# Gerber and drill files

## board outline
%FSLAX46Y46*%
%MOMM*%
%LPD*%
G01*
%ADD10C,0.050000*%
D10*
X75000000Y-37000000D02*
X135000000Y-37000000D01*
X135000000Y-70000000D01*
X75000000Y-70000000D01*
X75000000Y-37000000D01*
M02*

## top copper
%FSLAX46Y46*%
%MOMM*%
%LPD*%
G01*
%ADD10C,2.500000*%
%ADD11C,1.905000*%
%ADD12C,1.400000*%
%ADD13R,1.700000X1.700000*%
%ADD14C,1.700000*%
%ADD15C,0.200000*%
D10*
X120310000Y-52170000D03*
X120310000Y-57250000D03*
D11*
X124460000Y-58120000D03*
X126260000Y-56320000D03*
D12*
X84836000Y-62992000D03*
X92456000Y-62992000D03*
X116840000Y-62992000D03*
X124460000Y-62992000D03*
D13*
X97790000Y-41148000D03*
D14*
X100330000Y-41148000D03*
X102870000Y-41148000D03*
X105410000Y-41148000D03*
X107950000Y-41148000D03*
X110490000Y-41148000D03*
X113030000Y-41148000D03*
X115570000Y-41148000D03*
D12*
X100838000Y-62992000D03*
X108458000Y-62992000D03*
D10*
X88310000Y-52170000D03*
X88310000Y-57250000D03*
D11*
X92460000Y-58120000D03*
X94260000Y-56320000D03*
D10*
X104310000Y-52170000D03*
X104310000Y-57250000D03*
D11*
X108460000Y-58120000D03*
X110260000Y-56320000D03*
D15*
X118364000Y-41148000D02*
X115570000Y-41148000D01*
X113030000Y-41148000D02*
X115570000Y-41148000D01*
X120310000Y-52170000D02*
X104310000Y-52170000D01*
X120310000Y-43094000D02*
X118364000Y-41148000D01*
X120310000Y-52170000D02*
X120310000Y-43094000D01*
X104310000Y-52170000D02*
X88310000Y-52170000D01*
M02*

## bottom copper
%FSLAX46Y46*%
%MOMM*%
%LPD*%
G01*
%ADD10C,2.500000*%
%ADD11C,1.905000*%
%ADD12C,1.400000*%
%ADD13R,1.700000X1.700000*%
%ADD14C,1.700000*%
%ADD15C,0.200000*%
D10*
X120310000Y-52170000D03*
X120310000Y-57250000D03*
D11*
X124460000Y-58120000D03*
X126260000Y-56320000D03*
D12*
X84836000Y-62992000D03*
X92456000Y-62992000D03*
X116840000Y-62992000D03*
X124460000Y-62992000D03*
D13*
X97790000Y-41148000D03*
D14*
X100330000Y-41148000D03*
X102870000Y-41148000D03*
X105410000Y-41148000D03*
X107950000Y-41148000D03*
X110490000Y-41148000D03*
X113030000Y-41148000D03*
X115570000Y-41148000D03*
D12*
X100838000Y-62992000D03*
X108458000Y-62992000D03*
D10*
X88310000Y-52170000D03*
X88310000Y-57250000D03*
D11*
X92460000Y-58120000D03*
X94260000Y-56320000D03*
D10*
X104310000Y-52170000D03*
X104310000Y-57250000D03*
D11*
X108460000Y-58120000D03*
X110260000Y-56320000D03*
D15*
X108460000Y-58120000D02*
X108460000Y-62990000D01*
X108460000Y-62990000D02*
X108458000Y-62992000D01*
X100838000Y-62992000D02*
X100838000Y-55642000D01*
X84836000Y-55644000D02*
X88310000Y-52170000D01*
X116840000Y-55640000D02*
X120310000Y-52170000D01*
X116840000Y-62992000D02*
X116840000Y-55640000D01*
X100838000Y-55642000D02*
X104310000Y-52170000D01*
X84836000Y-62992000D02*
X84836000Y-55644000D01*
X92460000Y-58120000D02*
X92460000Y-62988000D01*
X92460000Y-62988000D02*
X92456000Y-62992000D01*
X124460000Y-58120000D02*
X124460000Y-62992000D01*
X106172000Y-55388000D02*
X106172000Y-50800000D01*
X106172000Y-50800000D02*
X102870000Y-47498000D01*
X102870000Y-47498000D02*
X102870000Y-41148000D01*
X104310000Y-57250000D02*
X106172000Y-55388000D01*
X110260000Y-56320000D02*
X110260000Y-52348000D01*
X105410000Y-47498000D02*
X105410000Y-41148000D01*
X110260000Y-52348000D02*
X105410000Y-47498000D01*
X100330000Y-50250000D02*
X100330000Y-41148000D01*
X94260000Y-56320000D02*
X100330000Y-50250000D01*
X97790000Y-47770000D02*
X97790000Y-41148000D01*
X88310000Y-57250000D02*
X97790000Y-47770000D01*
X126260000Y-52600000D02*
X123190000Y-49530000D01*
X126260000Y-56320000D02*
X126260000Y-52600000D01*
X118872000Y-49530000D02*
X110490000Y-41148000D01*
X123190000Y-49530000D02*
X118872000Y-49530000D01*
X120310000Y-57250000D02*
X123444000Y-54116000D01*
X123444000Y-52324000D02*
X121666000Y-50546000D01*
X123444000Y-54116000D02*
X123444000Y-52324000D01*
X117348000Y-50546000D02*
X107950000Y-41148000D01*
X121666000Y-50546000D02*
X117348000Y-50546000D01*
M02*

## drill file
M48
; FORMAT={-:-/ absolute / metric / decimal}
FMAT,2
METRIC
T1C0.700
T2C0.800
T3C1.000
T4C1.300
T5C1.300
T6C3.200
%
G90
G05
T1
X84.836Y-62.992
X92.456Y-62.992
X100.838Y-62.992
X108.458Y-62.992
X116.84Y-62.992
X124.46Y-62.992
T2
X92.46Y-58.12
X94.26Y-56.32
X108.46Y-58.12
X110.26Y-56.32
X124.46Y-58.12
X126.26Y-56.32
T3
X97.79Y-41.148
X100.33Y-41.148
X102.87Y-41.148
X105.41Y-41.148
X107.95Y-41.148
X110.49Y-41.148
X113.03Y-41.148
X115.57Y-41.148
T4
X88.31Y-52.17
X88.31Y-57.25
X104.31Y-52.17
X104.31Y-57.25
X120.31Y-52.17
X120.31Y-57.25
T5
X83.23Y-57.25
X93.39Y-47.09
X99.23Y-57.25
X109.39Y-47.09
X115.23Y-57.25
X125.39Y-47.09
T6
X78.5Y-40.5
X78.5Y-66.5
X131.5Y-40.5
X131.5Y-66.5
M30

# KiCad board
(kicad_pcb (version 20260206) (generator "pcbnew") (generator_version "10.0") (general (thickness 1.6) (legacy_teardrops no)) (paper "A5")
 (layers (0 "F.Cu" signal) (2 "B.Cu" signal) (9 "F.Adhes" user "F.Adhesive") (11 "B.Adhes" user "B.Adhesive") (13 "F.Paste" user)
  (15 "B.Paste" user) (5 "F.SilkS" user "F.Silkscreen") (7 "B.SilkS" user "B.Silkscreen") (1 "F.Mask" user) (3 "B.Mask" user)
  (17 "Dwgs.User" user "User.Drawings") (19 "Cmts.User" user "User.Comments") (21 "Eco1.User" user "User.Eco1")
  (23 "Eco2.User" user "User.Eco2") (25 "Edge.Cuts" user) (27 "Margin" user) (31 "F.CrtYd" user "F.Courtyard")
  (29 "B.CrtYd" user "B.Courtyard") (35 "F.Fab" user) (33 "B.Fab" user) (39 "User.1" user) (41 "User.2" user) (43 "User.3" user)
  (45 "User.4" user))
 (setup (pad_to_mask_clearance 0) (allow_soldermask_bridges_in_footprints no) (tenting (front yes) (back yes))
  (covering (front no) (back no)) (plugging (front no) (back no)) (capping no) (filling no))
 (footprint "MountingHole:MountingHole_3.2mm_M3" (layer "F.Cu") (at 78.5 40.5)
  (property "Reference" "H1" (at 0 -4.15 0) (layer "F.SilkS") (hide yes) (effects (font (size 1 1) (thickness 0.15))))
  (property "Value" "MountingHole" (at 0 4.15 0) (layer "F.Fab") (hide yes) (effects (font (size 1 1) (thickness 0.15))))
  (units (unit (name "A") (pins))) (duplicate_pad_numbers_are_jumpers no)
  (pad "" np_thru_hole circle (at 0 0) (size 3.2 3.2) (drill 3.2) (layers "*.Cu" "*.Mask")))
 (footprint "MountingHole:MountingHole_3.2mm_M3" (layer "F.Cu") (at 131.5 66.5)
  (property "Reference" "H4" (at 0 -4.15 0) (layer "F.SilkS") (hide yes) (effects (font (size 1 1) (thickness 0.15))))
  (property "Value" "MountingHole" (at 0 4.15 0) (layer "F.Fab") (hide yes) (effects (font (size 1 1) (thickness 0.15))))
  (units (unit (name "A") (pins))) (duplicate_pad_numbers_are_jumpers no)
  (pad "" np_thru_hole circle (at 0 0) (size 3.2 3.2) (drill 3.2) (layers "*.Cu" "*.Mask")))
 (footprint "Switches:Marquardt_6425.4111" (layer "F.Cu") (at 120.31 52.17 180)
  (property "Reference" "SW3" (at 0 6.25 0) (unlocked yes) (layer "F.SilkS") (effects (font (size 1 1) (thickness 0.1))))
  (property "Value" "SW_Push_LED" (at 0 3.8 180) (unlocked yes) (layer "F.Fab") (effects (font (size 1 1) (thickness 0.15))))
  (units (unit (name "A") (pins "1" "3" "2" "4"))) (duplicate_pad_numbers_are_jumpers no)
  (pad "" np_thru_hole circle (at -5.08 5.08 180) (size 1.3 1.3) (drill 1.3) (layers "*.Cu" "*.Mask"))
  (pad "" np_thru_hole circle (at 5.08 -5.08 180) (size 1.3 1.3) (drill 1.3) (layers "*.Cu" "*.Mask"))
  (pad "1" thru_hole circle (at 0 0 180) (size 2.5 2.5) (drill 1.3) (layers "*.Cu" "*.Mask") (remove_unused_layers no) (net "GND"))
  (pad "2" thru_hole circle (at 0 -5.08 180) (size 2.5 2.5) (drill 1.3) (layers "*.Cu" "*.Mask") (remove_unused_layers no)
   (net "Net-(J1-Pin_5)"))
  (pad "3" thru_hole circle (at -4.15 -5.95 180) (size 1.905 1.905) (drill 0.8) (layers "*.Cu" "*.Mask") (remove_unused_layers no)
   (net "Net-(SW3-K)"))
  (pad "4" thru_hole circle (at -5.95 -4.15 180) (size 1.905 1.905) (drill 0.8) (layers "*.Cu" "*.Mask") (remove_unused_layers no)
   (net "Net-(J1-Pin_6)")))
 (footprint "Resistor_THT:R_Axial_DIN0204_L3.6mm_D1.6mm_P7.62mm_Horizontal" (layer "F.Cu") (at 84.836 62.992)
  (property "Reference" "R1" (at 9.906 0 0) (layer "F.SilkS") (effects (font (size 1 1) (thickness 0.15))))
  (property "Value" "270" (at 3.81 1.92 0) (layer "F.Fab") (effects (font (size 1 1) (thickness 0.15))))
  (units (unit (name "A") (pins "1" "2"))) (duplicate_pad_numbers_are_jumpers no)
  (pad "1" thru_hole circle (at 0 0) (size 1.4 1.4) (drill 0.7) (layers "*.Cu" "*.Mask") (remove_unused_layers no) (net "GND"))
  (pad "2" thru_hole circle (at 7.62 0) (size 1.4 1.4) (drill 0.7) (layers "*.Cu" "*.Mask") (remove_unused_layers no) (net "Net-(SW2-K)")))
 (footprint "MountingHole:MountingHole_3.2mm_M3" (layer "F.Cu") (at 131.5 40.5)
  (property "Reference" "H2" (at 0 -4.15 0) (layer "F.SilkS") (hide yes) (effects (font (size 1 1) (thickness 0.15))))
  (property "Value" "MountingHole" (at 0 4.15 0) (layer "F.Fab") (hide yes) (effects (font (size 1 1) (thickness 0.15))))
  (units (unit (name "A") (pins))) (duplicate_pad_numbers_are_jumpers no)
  (pad "" np_thru_hole circle (at 0 0) (size 3.2 3.2) (drill 3.2) (layers "*.Cu" "*.Mask")))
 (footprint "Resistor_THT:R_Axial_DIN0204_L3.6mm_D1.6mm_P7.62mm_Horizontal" (layer "F.Cu") (at 116.84 62.992)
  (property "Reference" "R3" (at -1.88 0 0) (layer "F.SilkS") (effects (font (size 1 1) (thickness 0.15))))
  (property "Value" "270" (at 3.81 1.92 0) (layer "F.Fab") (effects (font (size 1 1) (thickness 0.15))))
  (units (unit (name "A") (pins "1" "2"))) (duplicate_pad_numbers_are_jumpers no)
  (pad "1" thru_hole circle (at 0 0) (size 1.4 1.4) (drill 0.7) (layers "*.Cu" "*.Mask") (remove_unused_layers no) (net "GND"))
  (pad "2" thru_hole circle (at 7.62 0) (size 1.4 1.4) (drill 0.7) (layers "*.Cu" "*.Mask") (remove_unused_layers no) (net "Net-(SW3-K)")))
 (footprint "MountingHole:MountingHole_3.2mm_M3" (layer "F.Cu") (at 78.5 66.5)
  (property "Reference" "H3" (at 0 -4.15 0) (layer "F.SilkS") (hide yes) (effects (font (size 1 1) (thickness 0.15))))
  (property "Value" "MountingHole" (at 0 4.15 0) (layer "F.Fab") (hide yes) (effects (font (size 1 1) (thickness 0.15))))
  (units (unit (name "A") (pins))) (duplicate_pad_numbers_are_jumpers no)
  (pad "" np_thru_hole circle (at 0 0) (size 3.2 3.2) (drill 3.2) (layers "*.Cu" "*.Mask")))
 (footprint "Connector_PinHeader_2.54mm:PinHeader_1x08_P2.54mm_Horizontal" (layer "F.Cu") (at 97.79 41.148 90)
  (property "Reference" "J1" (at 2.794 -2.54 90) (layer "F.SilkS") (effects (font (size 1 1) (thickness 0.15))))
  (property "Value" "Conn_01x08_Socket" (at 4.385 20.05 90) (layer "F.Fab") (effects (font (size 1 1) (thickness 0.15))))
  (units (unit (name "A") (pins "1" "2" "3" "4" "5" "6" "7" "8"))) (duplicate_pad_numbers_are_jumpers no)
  (pad "1" thru_hole rect (at 0 0 90) (size 1.7 1.7) (drill 1) (layers "*.Cu" "*.Mask") (remove_unused_layers no) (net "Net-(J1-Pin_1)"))
  (pad "2" thru_hole circle (at 0 2.54 90) (size 1.7 1.7) (drill 1) (layers "*.Cu" "*.Mask") (remove_unused_layers no)
   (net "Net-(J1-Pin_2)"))
  (pad "3" thru_hole circle (at 0 5.08 90) (size 1.7 1.7) (drill 1) (layers "*.Cu" "*.Mask") (remove_unused_layers no)
   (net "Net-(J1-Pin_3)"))
  (pad "4" thru_hole circle (at 0 7.62 90) (size 1.7 1.7) (drill 1) (layers "*.Cu" "*.Mask") (remove_unused_layers no)
   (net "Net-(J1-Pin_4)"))
  (pad "5" thru_hole circle (at 0 10.16 90) (size 1.7 1.7) (drill 1) (layers "*.Cu" "*.Mask") (remove_unused_layers no)
   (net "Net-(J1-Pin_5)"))
  (pad "6" thru_hole circle (at 0 12.7 90) (size 1.7 1.7) (drill 1) (layers "*.Cu" "*.Mask") (remove_unused_layers no)
   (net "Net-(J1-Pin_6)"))
  (pad "7" thru_hole circle (at 0 15.24 90) (size 1.7 1.7) (drill 1) (layers "*.Cu" "*.Mask") (remove_unused_layers no) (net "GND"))
  (pad "8" thru_hole circle (at 0 17.78 90) (size 1.7 1.7) (drill 1) (layers "*.Cu" "*.Mask") (remove_unused_layers no) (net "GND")))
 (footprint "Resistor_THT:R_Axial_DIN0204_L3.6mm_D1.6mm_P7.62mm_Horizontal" (layer "F.Cu") (at 100.838 62.992)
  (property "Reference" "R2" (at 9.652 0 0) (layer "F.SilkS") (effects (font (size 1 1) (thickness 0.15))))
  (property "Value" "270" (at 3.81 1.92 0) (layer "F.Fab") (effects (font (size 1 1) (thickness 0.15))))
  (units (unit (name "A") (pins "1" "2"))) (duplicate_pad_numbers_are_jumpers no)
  (pad "1" thru_hole circle (at 0 0) (size 1.4 1.4) (drill 0.7) (layers "*.Cu" "*.Mask") (remove_unused_layers no) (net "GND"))
  (pad "2" thru_hole circle (at 7.62 0) (size 1.4 1.4) (drill 0.7) (layers "*.Cu" "*.Mask") (remove_unused_layers no) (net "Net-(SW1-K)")))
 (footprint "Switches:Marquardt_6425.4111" (layer "F.Cu") (at 88.31 52.17 180)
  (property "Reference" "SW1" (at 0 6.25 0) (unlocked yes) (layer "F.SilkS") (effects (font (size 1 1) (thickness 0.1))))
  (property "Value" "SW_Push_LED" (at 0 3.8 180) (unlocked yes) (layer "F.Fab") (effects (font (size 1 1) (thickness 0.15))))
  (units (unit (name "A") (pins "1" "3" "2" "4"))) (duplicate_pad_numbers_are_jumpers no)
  (pad "" np_thru_hole circle (at -5.08 5.08 180) (size 1.3 1.3) (drill 1.3) (layers "*.Cu" "*.Mask"))
  (pad "" np_thru_hole circle (at 5.08 -5.08 180) (size 1.3 1.3) (drill 1.3) (layers "*.Cu" "*.Mask"))
  (pad "1" thru_hole circle (at 0 0 180) (size 2.5 2.5) (drill 1.3) (layers "*.Cu" "*.Mask") (remove_unused_layers no) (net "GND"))
  (pad "2" thru_hole circle (at 0 -5.08 180) (size 2.5 2.5) (drill 1.3) (layers "*.Cu" "*.Mask") (remove_unused_layers no)
   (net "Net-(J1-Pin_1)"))
  (pad "3" thru_hole circle (at -4.15 -5.95 180) (size 1.905 1.905) (drill 0.8) (layers "*.Cu" "*.Mask") (remove_unused_layers no)
   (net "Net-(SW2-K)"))
  (pad "4" thru_hole circle (at -5.95 -4.15 180) (size 1.905 1.905) (drill 0.8) (layers "*.Cu" "*.Mask") (remove_unused_layers no)
   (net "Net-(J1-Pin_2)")))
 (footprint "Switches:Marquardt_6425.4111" (layer "F.Cu") (at 104.31 52.17 180)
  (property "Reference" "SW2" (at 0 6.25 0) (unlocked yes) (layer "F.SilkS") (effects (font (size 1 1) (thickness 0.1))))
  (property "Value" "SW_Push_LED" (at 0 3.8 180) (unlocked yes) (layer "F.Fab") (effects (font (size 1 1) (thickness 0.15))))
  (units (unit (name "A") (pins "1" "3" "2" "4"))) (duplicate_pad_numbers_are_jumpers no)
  (pad "" np_thru_hole circle (at -5.08 5.08 180) (size 1.3 1.3) (drill 1.3) (layers "*.Cu" "*.Mask"))
  (pad "" np_thru_hole circle (at 5.08 -5.08 180) (size 1.3 1.3) (drill 1.3) (layers "*.Cu" "*.Mask"))
  (pad "1" thru_hole circle (at 0 0 180) (size 2.5 2.5) (drill 1.3) (layers "*.Cu" "*.Mask") (remove_unused_layers no) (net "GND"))
  (pad "2" thru_hole circle (at 0 -5.08 180) (size 2.5 2.5) (drill 1.3) (layers "*.Cu" "*.Mask") (remove_unused_layers no)
   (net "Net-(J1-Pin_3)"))
  (pad "3" thru_hole circle (at -4.15 -5.95 180) (size 1.905 1.905) (drill 0.8) (layers "*.Cu" "*.Mask") (remove_unused_layers no)
   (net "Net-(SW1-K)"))
  (pad "4" thru_hole circle (at -5.95 -4.15 180) (size 1.905 1.905) (drill 0.8) (layers "*.Cu" "*.Mask") (remove_unused_layers no)
   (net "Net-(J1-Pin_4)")))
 (gr_rect (start 75 37) (end 135 70) (stroke (width 0.05) (type default)) (fill no) (layer "Edge.Cuts"))
 (segment (start 108.46 58.12) (end 108.46 62.99) (width 0.2) (layer "B.Cu") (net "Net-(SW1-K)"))
 (segment (start 108.46 62.99) (end 108.458 62.992) (width 0.2) (layer "B.Cu") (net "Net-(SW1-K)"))
 (segment (start 118.364 41.148) (end 115.57 41.148) (width 0.2) (layer "F.Cu") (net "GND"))
 (segment (start 113.03 41.148) (end 115.57 41.148) (width 0.2) (layer "F.Cu") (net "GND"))
 (segment (start 120.31 52.17) (end 104.31 52.17) (width 0.2) (layer "F.Cu") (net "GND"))
 (segment (start 120.31 43.094) (end 118.364 41.148) (width 0.2) (layer "F.Cu") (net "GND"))
 (segment (start 120.31 52.17) (end 120.31 43.094) (width 0.2) (layer "F.Cu") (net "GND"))
 (segment (start 104.31 52.17) (end 88.31 52.17) (width 0.2) (layer "F.Cu") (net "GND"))
 (segment (start 100.838 62.992) (end 100.838 55.642) (width 0.2) (layer "B.Cu") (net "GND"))
 (segment (start 84.836 55.644) (end 88.31 52.17) (width 0.2) (layer "B.Cu") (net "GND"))
 (segment (start 116.84 55.64) (end 120.31 52.17) (width 0.2) (layer "B.Cu") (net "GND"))
 (segment (start 116.84 62.992) (end 116.84 55.64) (width 0.2) (layer "B.Cu") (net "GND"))
 (segment (start 100.838 55.642) (end 104.31 52.17) (width 0.2) (layer "B.Cu") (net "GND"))
 (segment (start 84.836 62.992) (end 84.836 55.644) (width 0.2) (layer "B.Cu") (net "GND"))
 (segment (start 92.46 58.12) (end 92.46 62.988) (width 0.2) (layer "B.Cu") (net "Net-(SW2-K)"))
 (segment (start 92.46 62.988) (end 92.456 62.992) (width 0.2) (layer "B.Cu") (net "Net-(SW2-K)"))
 (segment (start 124.46 58.12) (end 124.46 62.992) (width 0.2) (layer "B.Cu") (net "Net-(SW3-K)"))
 (segment (start 106.172 55.388) (end 106.172 50.8) (width 0.2) (layer "B.Cu") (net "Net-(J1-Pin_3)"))
 (segment (start 106.172 50.8) (end 102.87 47.498) (width 0.2) (layer "B.Cu") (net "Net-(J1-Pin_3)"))
 (segment (start 102.87 47.498) (end 102.87 41.148) (width 0.2) (layer "B.Cu") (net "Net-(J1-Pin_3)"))
 (segment (start 104.31 57.25) (end 106.172 55.388) (width 0.2) (layer "B.Cu") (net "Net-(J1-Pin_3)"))
 (segment (start 110.26 56.32) (end 110.26 52.348) (width 0.2) (layer "B.Cu") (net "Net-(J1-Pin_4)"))
 (segment (start 105.41 47.498) (end 105.41 41.148) (width 0.2) (layer "B.Cu") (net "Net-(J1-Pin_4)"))
 (segment (start 110.26 52.348) (end 105.41 47.498) (width 0.2) (layer "B.Cu") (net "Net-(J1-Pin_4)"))
 (segment (start 100.33 50.25) (end 100.33 41.148) (width 0.2) (layer "B.Cu") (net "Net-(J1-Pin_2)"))
 (segment (start 94.26 56.32) (end 100.33 50.25) (width 0.2) (layer "B.Cu") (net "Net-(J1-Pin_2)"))
 (segment (start 97.79 47.77) (end 97.79 41.148) (width 0.2) (layer "B.Cu") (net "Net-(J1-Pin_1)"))
 (segment (start 88.31 57.25) (end 97.79 47.77) (width 0.2) (layer "B.Cu") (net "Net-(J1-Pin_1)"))
 (segment (start 126.26 52.6) (end 123.19 49.53) (width 0.2) (layer "B.Cu") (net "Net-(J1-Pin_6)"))
 (segment (start 126.26 56.32) (end 126.26 52.6) (width 0.2) (layer "B.Cu") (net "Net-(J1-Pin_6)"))
 (segment (start 118.872 49.53) (end 110.49 41.148) (width 0.2) (layer "B.Cu") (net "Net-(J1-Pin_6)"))
 (segment (start 123.19 49.53) (end 118.872 49.53) (width 0.2) (layer "B.Cu") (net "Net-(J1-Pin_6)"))
 (segment (start 120.31 57.25) (end 123.444 54.116) (width 0.2) (layer "B.Cu") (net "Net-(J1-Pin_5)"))
 (segment (start 123.444 52.324) (end 121.666 50.546) (width 0.2) (layer "B.Cu") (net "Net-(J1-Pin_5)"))
 (segment (start 123.444 54.116) (end 123.444 52.324) (width 0.2) (layer "B.Cu") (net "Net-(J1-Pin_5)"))
 (segment (start 117.348 50.546) (end 107.95 41.148) (width 0.2) (layer "B.Cu") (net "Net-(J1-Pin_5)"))
 (segment (start 121.666 50.546) (end 117.348 50.546) (width 0.2) (layer "B.Cu") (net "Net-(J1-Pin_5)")))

